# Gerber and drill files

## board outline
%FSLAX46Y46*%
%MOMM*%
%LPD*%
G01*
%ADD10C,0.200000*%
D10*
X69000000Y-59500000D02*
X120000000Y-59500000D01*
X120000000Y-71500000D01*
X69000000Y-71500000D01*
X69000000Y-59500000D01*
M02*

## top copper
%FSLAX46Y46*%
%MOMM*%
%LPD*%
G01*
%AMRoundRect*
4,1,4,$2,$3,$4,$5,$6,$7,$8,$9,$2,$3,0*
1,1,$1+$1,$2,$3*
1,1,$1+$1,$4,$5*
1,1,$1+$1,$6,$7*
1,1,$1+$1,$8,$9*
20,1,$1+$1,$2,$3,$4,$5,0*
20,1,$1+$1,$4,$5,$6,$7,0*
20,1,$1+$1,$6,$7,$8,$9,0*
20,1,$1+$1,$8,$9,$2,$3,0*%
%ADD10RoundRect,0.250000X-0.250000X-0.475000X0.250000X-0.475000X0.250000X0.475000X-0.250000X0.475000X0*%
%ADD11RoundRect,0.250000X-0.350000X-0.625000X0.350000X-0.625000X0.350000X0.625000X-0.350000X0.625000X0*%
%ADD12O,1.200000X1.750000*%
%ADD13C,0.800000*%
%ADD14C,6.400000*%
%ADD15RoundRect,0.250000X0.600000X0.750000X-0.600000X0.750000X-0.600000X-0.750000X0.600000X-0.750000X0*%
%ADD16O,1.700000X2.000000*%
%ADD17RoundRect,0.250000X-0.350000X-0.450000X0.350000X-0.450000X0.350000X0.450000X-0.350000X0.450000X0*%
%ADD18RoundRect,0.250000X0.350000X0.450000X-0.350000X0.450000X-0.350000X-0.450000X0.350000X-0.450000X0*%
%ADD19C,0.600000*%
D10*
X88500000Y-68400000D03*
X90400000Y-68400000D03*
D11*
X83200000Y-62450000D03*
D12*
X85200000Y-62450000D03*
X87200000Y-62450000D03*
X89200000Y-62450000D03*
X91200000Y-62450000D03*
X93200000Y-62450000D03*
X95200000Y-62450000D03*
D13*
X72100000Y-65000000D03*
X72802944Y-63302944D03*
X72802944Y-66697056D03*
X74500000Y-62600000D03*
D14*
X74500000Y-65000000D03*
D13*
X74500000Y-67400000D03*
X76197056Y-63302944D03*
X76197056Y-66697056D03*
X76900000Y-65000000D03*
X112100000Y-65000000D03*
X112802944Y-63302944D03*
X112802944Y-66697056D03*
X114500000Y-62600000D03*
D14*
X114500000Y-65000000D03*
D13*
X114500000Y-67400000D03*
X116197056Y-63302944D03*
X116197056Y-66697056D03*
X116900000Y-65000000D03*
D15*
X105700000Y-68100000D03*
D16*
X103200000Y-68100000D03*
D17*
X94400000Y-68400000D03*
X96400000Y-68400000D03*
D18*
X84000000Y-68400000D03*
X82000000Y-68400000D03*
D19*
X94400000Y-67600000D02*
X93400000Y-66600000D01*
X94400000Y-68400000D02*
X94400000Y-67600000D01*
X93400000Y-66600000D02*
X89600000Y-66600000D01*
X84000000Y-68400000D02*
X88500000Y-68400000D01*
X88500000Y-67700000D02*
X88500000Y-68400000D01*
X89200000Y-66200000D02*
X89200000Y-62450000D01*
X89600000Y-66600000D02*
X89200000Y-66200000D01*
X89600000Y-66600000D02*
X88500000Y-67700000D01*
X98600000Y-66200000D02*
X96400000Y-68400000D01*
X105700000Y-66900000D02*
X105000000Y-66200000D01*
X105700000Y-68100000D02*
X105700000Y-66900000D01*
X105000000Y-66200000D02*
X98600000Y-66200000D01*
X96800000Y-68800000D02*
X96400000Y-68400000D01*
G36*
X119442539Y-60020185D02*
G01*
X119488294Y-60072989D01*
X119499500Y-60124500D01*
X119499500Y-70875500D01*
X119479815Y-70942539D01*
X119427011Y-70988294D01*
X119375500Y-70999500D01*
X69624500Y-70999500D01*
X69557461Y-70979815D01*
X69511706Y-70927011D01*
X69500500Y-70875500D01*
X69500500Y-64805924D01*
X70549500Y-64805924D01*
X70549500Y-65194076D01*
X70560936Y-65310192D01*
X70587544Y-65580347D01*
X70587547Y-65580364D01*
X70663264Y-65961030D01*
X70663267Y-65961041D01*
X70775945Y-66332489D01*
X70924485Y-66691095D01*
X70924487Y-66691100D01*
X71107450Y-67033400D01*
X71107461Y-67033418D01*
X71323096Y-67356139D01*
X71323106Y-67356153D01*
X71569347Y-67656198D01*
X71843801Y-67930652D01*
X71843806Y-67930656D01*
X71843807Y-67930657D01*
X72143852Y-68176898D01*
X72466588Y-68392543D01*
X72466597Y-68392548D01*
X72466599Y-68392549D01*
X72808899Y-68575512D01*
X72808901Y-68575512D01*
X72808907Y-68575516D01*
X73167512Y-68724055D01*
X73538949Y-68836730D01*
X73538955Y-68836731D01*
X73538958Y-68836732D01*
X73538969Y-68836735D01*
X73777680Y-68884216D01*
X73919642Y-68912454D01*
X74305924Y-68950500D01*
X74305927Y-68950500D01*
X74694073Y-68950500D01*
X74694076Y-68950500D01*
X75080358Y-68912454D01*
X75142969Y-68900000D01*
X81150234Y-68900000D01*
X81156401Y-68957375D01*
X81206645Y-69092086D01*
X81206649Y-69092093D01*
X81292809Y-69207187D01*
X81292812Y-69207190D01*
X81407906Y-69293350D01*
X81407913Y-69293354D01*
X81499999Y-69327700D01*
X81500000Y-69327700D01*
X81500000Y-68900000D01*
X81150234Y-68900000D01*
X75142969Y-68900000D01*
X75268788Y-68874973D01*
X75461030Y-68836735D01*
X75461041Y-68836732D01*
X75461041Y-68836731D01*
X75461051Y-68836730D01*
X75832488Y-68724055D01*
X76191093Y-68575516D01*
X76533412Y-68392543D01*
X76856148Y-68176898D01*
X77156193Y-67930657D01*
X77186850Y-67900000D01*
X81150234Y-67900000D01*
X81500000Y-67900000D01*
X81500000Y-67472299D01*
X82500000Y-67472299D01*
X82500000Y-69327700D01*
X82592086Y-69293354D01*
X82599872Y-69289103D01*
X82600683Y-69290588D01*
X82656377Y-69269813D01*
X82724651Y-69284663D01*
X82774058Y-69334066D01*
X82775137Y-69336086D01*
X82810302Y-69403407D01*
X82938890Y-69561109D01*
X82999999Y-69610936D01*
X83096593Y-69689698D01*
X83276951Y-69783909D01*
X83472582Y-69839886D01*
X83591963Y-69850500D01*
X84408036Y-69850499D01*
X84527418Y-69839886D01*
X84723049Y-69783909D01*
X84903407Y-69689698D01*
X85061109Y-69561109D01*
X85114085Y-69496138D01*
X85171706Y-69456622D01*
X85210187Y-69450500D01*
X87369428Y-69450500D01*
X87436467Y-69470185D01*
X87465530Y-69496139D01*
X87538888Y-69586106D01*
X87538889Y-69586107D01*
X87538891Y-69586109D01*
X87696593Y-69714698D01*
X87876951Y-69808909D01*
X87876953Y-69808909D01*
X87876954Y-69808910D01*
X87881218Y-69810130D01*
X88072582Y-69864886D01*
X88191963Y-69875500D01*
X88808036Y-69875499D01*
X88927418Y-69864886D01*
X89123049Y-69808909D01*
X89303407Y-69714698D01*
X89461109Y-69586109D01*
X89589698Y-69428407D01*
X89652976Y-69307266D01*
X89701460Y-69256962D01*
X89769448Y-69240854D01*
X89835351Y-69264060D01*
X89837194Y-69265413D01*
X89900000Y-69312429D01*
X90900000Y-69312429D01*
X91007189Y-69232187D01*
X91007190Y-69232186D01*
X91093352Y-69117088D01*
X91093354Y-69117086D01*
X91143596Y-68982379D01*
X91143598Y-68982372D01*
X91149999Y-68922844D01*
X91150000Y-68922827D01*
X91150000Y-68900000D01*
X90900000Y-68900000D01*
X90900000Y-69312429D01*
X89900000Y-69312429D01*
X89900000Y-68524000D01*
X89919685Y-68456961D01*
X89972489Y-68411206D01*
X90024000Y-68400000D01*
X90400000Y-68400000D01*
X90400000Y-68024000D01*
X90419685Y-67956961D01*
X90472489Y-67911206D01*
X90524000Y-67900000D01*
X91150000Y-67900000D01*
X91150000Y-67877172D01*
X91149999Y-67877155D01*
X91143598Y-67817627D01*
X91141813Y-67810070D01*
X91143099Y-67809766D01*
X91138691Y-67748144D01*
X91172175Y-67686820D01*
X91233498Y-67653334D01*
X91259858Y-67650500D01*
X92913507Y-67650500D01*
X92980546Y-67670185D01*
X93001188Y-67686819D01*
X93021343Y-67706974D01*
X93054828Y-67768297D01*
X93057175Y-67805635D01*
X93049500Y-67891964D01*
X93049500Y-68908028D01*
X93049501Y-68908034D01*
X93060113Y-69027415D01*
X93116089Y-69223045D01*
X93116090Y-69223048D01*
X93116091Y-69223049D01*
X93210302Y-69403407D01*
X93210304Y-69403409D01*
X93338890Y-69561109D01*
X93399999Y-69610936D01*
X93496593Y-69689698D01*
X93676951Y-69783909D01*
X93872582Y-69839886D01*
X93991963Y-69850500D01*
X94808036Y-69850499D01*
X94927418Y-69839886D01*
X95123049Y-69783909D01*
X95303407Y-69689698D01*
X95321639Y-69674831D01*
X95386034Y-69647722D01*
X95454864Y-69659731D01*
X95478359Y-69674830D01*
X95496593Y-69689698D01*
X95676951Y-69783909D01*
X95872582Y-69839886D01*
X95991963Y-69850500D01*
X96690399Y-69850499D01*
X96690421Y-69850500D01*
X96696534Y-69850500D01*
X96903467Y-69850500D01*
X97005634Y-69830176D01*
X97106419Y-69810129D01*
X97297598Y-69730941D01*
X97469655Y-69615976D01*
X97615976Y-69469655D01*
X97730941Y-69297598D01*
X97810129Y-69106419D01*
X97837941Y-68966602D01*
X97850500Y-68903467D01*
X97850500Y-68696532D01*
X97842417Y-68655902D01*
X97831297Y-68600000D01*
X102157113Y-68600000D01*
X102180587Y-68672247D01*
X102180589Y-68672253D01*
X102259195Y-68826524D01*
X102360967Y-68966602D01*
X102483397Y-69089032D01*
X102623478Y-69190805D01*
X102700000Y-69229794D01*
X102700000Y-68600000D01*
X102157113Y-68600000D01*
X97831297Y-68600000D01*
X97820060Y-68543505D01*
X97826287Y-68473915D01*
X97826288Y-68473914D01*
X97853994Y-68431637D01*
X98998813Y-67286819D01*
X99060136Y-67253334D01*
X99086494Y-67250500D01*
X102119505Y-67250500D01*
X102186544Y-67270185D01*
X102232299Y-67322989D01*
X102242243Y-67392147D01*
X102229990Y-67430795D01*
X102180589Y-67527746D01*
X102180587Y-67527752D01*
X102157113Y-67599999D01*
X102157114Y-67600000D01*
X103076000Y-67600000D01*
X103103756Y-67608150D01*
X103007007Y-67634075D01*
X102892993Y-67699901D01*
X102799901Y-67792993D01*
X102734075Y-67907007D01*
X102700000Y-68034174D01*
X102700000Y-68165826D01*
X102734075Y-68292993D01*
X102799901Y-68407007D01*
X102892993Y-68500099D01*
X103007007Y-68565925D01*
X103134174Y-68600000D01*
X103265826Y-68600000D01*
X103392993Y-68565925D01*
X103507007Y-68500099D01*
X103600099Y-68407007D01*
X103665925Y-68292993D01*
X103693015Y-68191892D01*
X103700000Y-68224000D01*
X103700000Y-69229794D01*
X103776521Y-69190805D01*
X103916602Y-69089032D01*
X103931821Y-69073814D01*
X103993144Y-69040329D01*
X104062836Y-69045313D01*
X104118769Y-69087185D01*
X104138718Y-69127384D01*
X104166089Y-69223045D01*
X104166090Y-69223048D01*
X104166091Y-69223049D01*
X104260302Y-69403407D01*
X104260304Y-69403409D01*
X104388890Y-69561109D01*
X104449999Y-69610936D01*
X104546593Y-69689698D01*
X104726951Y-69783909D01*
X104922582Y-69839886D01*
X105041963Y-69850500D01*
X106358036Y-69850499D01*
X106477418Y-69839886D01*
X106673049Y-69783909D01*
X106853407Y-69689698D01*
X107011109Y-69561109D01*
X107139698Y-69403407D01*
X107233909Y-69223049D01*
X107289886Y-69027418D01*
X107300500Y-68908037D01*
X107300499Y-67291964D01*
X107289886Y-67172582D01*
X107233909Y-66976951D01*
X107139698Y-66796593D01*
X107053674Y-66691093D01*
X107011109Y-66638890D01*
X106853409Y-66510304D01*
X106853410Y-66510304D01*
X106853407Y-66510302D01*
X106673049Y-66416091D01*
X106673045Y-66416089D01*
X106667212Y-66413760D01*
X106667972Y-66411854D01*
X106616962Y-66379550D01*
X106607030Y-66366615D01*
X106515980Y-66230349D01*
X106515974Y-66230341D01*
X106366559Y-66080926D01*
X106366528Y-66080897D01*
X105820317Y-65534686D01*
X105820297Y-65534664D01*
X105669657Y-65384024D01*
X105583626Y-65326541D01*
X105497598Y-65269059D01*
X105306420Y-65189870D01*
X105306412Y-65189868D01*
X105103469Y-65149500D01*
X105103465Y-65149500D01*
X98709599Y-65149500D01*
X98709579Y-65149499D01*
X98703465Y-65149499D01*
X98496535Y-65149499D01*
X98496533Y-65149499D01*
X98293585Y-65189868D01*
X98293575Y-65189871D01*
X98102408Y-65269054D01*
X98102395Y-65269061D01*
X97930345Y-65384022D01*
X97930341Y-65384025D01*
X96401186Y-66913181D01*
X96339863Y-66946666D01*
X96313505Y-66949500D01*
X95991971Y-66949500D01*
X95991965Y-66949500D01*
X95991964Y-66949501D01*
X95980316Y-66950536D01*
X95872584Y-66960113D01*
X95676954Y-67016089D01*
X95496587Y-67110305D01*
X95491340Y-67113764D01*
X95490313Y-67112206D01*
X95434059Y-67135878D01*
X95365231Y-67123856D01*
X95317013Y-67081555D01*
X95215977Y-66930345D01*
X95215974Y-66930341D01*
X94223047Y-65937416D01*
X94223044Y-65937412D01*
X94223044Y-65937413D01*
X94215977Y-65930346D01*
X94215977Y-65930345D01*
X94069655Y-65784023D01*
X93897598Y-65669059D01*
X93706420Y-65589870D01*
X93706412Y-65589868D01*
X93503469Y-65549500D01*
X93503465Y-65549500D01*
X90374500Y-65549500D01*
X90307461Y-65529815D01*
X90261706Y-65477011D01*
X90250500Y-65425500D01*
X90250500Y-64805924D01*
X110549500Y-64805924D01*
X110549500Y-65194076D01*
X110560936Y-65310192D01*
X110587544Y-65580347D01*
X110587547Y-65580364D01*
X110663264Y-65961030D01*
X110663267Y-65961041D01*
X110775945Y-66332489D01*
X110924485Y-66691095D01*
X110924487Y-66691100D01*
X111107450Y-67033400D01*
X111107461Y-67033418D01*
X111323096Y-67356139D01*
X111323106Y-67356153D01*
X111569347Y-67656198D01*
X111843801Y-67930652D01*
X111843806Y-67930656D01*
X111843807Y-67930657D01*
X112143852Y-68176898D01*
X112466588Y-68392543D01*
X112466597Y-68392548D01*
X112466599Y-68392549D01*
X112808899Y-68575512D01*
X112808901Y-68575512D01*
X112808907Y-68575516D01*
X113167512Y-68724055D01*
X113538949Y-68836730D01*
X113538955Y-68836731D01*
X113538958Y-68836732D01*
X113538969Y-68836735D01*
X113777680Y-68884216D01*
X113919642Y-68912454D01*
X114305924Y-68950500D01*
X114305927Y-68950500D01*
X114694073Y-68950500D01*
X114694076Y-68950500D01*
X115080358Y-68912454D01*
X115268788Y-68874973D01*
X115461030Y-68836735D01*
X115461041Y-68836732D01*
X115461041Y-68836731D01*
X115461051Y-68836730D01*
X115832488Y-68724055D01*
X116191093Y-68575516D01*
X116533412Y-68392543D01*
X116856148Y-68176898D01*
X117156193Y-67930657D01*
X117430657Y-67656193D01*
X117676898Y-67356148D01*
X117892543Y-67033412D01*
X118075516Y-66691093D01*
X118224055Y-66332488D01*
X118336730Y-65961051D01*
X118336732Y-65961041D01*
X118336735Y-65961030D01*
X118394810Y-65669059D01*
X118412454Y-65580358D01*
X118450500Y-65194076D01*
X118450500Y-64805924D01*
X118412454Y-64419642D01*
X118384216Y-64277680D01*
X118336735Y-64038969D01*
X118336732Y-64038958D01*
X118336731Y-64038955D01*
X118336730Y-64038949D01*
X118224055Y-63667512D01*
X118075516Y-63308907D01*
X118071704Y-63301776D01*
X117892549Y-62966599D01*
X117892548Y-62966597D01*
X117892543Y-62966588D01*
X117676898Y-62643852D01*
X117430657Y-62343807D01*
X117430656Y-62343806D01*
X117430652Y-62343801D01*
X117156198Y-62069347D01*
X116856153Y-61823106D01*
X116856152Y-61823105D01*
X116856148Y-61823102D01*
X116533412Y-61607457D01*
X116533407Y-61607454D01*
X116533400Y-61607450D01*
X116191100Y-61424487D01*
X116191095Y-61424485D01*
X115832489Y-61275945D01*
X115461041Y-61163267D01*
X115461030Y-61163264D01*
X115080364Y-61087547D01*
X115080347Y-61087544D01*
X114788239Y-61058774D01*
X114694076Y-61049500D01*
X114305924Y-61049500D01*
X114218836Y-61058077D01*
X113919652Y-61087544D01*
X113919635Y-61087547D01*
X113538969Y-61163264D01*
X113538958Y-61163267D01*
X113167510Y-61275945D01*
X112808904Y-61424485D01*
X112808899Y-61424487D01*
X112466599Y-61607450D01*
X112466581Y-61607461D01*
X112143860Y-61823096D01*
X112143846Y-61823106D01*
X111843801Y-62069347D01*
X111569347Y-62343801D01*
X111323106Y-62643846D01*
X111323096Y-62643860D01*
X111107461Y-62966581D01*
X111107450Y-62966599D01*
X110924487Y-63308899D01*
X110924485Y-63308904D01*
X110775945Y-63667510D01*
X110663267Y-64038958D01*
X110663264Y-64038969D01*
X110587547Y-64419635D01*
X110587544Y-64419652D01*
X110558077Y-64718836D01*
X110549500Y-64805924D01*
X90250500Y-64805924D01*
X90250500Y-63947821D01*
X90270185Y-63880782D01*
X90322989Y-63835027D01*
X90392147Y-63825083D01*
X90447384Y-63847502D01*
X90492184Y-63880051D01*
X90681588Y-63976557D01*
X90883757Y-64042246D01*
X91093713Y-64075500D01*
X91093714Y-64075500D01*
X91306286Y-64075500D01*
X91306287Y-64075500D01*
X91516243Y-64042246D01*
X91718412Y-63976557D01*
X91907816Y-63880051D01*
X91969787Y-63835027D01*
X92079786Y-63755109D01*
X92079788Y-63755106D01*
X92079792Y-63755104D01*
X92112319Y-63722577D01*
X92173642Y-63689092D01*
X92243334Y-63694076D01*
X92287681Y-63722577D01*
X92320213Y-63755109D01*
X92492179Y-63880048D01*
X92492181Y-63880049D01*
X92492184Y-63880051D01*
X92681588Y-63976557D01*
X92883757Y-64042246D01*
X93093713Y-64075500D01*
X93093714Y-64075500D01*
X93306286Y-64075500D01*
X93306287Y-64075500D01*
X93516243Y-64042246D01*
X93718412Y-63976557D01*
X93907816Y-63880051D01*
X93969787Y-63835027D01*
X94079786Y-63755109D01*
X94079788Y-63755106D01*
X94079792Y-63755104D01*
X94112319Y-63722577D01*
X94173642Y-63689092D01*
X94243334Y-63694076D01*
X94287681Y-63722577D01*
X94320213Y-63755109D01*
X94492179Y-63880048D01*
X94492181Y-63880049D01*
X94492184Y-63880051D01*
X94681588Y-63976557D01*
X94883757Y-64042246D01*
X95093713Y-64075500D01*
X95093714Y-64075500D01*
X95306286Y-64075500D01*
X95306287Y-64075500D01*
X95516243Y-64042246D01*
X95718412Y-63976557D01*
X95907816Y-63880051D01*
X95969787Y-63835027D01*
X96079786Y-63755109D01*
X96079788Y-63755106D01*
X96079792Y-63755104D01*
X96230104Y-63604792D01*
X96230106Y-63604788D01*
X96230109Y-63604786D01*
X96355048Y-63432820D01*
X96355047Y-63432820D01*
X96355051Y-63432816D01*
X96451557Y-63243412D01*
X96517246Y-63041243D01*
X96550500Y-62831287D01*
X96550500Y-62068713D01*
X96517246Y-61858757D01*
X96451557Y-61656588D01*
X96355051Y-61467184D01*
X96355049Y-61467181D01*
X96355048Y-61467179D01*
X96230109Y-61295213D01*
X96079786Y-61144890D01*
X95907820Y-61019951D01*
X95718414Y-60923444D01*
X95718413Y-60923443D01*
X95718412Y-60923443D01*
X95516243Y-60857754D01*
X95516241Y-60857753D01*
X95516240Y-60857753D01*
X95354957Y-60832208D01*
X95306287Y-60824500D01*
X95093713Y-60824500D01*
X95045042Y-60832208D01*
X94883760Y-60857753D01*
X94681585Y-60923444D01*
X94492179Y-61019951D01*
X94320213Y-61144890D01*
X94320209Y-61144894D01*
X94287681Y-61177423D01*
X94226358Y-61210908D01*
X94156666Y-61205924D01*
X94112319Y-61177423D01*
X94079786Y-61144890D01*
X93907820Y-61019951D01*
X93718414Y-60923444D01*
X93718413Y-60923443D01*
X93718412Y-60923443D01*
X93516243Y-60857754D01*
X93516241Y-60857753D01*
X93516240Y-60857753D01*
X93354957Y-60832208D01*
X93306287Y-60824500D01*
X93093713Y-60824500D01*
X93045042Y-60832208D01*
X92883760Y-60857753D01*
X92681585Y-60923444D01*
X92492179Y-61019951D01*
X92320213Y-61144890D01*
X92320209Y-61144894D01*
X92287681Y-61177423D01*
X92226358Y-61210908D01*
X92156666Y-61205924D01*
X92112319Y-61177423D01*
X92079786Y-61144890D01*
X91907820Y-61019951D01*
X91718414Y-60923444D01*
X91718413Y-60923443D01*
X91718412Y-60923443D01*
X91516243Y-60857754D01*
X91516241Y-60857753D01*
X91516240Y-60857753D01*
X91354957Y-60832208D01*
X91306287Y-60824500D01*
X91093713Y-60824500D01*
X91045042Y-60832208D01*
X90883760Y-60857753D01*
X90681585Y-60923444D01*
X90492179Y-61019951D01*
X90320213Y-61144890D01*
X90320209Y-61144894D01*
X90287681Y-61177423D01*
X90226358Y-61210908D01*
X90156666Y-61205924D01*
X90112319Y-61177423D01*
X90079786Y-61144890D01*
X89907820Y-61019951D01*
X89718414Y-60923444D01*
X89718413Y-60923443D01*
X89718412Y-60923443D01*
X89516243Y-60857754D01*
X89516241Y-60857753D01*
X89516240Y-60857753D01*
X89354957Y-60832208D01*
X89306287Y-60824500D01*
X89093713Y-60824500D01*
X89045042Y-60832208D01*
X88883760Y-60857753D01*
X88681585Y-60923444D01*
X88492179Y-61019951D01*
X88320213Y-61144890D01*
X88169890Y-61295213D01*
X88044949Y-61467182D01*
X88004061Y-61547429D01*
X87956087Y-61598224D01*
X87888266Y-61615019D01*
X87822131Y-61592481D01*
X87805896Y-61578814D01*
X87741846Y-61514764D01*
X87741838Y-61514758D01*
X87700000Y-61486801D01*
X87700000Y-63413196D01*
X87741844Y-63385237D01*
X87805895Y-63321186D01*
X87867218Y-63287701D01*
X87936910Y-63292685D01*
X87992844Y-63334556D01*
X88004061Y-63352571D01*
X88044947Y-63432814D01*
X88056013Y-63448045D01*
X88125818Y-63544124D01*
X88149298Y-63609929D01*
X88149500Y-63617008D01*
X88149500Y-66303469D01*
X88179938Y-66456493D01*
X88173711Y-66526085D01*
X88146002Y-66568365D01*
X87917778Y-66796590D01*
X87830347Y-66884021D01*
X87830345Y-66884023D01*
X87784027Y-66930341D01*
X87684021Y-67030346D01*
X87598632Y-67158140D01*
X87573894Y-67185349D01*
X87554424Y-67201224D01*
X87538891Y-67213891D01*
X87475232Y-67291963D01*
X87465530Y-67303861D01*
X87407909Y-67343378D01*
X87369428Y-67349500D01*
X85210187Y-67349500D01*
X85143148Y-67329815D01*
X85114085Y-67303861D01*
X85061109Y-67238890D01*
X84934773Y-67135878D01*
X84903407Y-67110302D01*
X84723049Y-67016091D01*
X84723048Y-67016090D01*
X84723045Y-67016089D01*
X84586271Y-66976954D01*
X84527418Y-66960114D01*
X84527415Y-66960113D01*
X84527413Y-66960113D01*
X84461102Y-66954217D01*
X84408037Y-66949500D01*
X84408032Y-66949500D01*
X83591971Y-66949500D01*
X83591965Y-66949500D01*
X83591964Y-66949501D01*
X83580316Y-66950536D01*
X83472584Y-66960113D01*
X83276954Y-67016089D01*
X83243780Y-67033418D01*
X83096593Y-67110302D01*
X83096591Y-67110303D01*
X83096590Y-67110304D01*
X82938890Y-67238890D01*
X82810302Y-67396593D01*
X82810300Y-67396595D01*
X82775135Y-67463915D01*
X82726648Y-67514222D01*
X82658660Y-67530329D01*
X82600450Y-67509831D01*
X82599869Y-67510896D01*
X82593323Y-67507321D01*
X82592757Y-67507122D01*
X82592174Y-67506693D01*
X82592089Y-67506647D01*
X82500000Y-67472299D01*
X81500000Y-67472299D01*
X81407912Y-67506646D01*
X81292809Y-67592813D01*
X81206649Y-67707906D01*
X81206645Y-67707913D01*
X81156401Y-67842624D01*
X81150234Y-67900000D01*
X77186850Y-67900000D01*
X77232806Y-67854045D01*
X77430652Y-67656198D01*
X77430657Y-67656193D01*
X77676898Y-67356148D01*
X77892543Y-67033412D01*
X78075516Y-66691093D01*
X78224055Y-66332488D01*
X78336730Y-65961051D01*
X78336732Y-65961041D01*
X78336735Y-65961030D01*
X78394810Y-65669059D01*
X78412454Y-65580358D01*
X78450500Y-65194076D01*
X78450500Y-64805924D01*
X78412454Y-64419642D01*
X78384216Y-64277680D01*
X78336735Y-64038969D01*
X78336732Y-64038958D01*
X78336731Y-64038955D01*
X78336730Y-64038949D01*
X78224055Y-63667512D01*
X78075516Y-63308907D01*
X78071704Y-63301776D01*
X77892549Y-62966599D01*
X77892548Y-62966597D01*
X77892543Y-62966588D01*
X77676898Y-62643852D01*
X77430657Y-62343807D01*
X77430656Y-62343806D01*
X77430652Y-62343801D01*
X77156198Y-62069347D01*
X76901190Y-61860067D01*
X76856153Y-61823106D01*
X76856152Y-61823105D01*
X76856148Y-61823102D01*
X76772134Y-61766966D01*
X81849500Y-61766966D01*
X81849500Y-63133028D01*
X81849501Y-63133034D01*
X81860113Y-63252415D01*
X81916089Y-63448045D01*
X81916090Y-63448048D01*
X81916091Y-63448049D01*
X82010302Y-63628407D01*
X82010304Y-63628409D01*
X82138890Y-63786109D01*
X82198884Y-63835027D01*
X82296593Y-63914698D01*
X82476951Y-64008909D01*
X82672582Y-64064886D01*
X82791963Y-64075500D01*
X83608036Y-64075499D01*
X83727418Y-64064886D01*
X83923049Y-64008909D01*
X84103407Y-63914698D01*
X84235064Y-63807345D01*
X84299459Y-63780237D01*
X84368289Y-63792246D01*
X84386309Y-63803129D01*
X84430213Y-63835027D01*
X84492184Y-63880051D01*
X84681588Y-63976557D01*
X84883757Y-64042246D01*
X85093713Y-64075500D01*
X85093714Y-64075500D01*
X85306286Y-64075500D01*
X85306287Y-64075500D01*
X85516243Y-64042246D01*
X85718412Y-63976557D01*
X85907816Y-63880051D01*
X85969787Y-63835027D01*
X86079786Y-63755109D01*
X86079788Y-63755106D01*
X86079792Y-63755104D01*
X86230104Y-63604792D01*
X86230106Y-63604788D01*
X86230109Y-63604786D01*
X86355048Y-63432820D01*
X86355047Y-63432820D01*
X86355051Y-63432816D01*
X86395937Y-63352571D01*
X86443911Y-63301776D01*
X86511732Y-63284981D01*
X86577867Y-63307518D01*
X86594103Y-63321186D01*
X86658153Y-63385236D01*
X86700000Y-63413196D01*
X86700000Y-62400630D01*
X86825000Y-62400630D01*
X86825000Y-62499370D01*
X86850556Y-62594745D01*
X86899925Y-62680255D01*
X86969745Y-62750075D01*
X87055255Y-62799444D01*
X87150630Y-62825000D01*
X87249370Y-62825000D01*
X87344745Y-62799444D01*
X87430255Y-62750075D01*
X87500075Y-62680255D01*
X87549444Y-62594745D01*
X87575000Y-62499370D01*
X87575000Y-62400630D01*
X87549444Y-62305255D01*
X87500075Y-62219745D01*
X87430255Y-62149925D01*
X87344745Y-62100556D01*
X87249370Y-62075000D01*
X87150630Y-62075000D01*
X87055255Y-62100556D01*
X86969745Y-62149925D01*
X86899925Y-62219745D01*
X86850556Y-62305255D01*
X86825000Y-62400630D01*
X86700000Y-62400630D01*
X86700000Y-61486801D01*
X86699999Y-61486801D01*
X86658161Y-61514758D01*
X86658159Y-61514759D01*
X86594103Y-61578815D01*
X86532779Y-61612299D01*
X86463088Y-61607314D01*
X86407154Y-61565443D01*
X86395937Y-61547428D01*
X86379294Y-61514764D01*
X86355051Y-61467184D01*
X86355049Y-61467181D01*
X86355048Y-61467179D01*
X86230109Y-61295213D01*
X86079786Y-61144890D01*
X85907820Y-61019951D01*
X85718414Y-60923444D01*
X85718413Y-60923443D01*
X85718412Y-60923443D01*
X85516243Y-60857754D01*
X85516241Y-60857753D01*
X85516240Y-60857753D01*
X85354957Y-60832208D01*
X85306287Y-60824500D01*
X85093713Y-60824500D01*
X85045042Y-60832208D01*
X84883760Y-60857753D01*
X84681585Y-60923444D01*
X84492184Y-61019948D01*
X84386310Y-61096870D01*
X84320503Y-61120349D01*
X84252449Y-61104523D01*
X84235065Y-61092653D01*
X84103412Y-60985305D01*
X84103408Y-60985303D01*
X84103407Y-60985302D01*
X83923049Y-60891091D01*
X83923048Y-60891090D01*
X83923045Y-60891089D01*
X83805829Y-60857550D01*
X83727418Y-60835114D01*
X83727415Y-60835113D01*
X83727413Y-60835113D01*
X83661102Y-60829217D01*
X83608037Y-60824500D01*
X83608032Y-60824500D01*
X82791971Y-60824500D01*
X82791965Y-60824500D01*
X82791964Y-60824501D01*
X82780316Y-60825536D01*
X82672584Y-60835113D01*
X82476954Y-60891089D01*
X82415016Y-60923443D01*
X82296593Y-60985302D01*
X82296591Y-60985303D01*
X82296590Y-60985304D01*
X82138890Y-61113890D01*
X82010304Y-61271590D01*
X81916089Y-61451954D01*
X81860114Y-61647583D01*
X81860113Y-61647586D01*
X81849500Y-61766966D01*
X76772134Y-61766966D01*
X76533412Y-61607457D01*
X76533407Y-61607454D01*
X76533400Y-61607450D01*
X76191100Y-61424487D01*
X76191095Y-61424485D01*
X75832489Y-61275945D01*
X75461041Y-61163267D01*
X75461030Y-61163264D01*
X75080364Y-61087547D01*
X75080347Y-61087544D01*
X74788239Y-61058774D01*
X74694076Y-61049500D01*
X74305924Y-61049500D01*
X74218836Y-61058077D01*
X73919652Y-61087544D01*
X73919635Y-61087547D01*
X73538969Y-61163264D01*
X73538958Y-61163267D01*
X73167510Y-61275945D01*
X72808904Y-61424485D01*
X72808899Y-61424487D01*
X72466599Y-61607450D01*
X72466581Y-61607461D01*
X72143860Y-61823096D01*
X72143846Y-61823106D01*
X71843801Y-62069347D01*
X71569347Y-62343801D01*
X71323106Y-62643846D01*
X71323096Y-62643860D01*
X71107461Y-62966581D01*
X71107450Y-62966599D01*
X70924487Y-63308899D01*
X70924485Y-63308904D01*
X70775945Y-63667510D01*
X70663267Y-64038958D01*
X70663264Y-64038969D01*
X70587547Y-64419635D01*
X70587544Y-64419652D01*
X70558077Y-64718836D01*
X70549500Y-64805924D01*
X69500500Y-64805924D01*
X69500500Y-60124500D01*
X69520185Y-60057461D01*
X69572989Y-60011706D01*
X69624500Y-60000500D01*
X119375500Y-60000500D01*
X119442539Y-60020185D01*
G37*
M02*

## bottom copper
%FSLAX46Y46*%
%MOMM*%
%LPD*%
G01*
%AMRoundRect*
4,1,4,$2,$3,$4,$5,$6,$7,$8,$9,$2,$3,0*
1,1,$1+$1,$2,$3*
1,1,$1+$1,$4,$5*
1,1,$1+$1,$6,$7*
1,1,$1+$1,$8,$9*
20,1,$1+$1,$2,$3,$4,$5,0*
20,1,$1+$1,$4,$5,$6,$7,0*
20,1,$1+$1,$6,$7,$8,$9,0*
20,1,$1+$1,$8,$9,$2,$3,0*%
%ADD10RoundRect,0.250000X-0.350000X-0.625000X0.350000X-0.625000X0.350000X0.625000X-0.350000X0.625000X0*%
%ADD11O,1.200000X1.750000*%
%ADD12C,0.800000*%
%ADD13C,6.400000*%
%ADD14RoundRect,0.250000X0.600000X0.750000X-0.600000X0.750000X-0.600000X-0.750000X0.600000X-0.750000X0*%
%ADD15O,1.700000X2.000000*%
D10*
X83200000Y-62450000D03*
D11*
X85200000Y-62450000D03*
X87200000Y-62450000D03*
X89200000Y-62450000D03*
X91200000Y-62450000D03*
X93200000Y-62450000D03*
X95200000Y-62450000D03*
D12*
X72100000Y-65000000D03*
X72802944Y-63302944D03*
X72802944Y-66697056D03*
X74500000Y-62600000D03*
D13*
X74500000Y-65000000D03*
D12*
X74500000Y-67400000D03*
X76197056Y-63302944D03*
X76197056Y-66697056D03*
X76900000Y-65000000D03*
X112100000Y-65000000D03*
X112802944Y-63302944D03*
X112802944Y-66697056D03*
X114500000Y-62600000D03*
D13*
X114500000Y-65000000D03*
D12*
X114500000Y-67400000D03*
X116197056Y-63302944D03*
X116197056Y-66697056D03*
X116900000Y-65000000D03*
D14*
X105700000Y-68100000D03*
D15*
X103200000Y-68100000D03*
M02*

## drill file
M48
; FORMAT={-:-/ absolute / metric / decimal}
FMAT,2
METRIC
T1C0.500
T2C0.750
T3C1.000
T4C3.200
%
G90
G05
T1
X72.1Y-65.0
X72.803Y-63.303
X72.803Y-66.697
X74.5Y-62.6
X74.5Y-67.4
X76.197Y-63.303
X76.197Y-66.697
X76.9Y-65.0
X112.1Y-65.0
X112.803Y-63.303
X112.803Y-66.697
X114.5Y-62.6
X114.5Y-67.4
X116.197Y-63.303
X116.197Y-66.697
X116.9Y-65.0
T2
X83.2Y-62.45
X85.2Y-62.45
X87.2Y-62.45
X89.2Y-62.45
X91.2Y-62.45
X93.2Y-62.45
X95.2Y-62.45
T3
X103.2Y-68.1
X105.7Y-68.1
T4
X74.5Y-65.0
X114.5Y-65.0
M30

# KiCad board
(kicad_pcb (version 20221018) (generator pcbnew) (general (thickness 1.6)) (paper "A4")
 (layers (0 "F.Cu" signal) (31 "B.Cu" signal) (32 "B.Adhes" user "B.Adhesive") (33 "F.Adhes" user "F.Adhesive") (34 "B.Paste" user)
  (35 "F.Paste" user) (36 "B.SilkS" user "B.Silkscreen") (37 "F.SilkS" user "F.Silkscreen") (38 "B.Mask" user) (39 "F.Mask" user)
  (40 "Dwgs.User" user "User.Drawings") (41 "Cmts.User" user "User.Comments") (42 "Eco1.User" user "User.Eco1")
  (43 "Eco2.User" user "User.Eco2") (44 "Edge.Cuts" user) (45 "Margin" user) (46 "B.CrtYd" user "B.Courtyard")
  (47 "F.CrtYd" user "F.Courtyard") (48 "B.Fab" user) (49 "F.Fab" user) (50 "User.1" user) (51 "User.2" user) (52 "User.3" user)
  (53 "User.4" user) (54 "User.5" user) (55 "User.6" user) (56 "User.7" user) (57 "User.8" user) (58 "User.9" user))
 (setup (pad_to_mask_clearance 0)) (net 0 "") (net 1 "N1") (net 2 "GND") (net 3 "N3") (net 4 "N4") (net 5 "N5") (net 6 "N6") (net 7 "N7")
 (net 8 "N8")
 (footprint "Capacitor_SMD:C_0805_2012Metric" (layer "F.Cu") (at 89.45 68.4)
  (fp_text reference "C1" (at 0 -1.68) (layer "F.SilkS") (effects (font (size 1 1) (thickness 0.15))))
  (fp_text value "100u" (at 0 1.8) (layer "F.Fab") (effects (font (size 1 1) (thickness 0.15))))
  (pad "1" smd roundrect (at -0.95 0) (size 1 1.45) (layers "F.Cu" "F.Paste" "F.Mask") (roundrect_rratio 0.25) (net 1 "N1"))
  (pad "2" smd roundrect (at 0.95 0) (size 1 1.45) (layers "F.Cu" "F.Paste" "F.Mask") (roundrect_rratio 0.25) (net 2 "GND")))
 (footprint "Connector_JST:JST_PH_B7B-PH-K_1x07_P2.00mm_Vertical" (layer "F.Cu") (at 83.2 62.45)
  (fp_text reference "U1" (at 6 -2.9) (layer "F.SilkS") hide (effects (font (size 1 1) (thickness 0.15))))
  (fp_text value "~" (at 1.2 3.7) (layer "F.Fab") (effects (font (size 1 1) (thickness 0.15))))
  (pad "1" thru_hole roundrect (at 0 0) (size 1.2 1.75) (drill 0.75) (layers "*.Cu" "*.Mask") (roundrect_rratio 0.208333) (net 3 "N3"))
  (pad "2" thru_hole oval (at 2 0) (size 1.2 1.75) (drill 0.75) (layers "*.Cu" "*.Mask") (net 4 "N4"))
  (pad "3" thru_hole oval (at 4 0) (size 1.2 1.75) (drill 0.75) (layers "*.Cu" "*.Mask") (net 2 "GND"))
  (pad "4" thru_hole oval (at 6 0) (size 1.2 1.75) (drill 0.75) (layers "*.Cu" "*.Mask") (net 1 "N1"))
  (pad "5" thru_hole oval (at 8 0) (size 1.2 1.75) (drill 0.75) (layers "*.Cu" "*.Mask") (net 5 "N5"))
  (pad "6" thru_hole oval (at 10 0) (size 1.2 1.75) (drill 0.75) (layers "*.Cu" "*.Mask") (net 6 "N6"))
  (pad "7" thru_hole oval (at 12 0) (size 1.2 1.75) (drill 0.75) (layers "*.Cu" "*.Mask") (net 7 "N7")))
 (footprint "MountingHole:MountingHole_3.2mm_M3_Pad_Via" (layer "F.Cu") (at 74.5 65)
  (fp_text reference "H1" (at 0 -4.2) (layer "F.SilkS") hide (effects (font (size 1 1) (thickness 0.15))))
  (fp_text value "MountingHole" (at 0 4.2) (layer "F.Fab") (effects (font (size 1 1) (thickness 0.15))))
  (pad "1" thru_hole circle (at -2.4 0) (size 0.8 0.8) (drill 0.5) (layers "*.Cu" "*.Mask"))
  (pad "1" thru_hole circle (at -1.697056 -1.697056) (size 0.8 0.8) (drill 0.5) (layers "*.Cu" "*.Mask"))
  (pad "1" thru_hole circle (at -1.697056 1.697056) (size 0.8 0.8) (drill 0.5) (layers "*.Cu" "*.Mask"))
  (pad "1" thru_hole circle (at 0 -2.4) (size 0.8 0.8) (drill 0.5) (layers "*.Cu" "*.Mask"))
  (pad "1" thru_hole circle (at 0 0) (size 6.4 6.4) (drill 3.2) (layers "*.Cu" "*.Mask"))
  (pad "1" thru_hole circle (at 0 2.4) (size 0.8 0.8) (drill 0.5) (layers "*.Cu" "*.Mask"))
  (pad "1" thru_hole circle (at 1.697056 -1.697056) (size 0.8 0.8) (drill 0.5) (layers "*.Cu" "*.Mask"))
  (pad "1" thru_hole circle (at 1.697056 1.697056) (size 0.8 0.8) (drill 0.5) (layers "*.Cu" "*.Mask"))
  (pad "1" thru_hole circle (at 2.4 0) (size 0.8 0.8) (drill 0.5) (layers "*.Cu" "*.Mask")))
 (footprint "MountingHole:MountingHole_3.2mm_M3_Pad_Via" (layer "F.Cu") (at 114.5 65)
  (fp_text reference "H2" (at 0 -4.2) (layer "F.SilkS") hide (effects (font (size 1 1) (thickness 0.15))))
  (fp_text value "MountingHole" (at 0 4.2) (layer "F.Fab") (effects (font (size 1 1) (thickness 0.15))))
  (pad "1" thru_hole circle (at -2.4 0) (size 0.8 0.8) (drill 0.5) (layers "*.Cu" "*.Mask"))
  (pad "1" thru_hole circle (at -1.697056 -1.697056) (size 0.8 0.8) (drill 0.5) (layers "*.Cu" "*.Mask"))
  (pad "1" thru_hole circle (at -1.697056 1.697056) (size 0.8 0.8) (drill 0.5) (layers "*.Cu" "*.Mask"))
  (pad "1" thru_hole circle (at 0 -2.4) (size 0.8 0.8) (drill 0.5) (layers "*.Cu" "*.Mask"))
  (pad "1" thru_hole circle (at 0 0) (size 6.4 6.4) (drill 3.2) (layers "*.Cu" "*.Mask"))
  (pad "1" thru_hole circle (at 0 2.4) (size 0.8 0.8) (drill 0.5) (layers "*.Cu" "*.Mask"))
  (pad "1" thru_hole circle (at 1.697056 -1.697056) (size 0.8 0.8) (drill 0.5) (layers "*.Cu" "*.Mask"))
  (pad "1" thru_hole circle (at 1.697056 1.697056) (size 0.8 0.8) (drill 0.5) (layers "*.Cu" "*.Mask"))
  (pad "1" thru_hole circle (at 2.4 0) (size 0.8 0.8) (drill 0.5) (layers "*.Cu" "*.Mask")))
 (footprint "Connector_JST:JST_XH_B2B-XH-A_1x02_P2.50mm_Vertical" (layer "F.Cu") (at 105.7 68.1 180)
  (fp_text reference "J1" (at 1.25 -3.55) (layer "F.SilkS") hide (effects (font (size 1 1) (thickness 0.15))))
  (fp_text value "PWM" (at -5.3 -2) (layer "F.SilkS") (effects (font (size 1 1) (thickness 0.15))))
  (pad "1" thru_hole roundrect (at 0 0 180) (size 1.7 2) (drill 1) (layers "*.Cu" "*.Mask") (roundrect_rratio 0.147059) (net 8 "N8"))
  (pad "2" thru_hole oval (at 2.5 0 180) (size 1.7 2) (drill 1) (layers "*.Cu" "*.Mask") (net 2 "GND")))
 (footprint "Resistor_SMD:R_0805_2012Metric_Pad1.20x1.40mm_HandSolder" (layer "F.Cu") (at 95.4 68.4)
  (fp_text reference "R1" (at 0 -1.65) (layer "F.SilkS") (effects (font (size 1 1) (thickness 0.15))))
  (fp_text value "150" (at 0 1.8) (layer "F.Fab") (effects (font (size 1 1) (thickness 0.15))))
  (pad "1" smd roundrect (at -1 0) (size 1.2 1.4) (layers "F.Cu" "F.Paste" "F.Mask") (roundrect_rratio 0.208333) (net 1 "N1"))
  (pad "2" smd roundrect (at 1 0) (size 1.2 1.4) (layers "F.Cu" "F.Paste" "F.Mask") (roundrect_rratio 0.208333) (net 8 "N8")))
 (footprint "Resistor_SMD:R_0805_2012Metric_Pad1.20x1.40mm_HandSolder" (layer "F.Cu") (at 83 68.4 180)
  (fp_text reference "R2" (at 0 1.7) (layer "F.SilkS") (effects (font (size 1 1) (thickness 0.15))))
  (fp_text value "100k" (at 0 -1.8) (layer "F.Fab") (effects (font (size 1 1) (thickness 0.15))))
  (pad "1" smd roundrect (at -1 0 180) (size 1.2 1.4) (layers "F.Cu" "F.Paste" "F.Mask") (roundrect_rratio 0.208333) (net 1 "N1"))
  (pad "2" smd roundrect (at 1 0 180) (size 1.2 1.4) (layers "F.Cu" "F.Paste" "F.Mask") (roundrect_rratio 0.208333) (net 2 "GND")))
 (gr_rect (start 69 59.5) (end 120 71.5) (stroke (width 0.2) (type default)) (fill none) (layer "Edge.Cuts"))
 (segment (start 94.4 67.6) (end 93.4 66.6) (width 0.6) (layer "F.Cu") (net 1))
 (segment (start 94.4 68.4) (end 94.4 67.6) (width 0.6) (layer "F.Cu") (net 1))
 (segment (start 93.4 66.6) (end 89.6 66.6) (width 0.6) (layer "F.Cu") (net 1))
 (segment (start 84 68.4) (end 88.5 68.4) (width 0.6) (layer "F.Cu") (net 1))
 (segment (start 88.5 67.7) (end 88.5 68.4) (width 0.6) (layer "F.Cu") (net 1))
 (segment (start 89.2 66.2) (end 89.2 62.45) (width 0.6) (layer "F.Cu") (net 1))
 (segment (start 89.6 66.6) (end 89.2 66.2) (width 0.6) (layer "F.Cu") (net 1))
 (segment (start 89.6 66.6) (end 88.5 67.7) (width 0.6) (layer "F.Cu") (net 1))
 (segment (start 98.6 66.2) (end 96.4 68.4) (width 0.6) (layer "F.Cu") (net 8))
 (segment (start 105.7 66.9) (end 105 66.2) (width 0.6) (layer "F.Cu") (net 8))
 (segment (start 105.7 68.1) (end 105.7 66.9) (width 0.6) (layer "F.Cu") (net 8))
 (segment (start 105 66.2) (end 98.6 66.2) (width 0.6) (layer "F.Cu") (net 8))
 (segment (start 96.8 68.8) (end 96.4 68.4) (width 0.6) (layer "F.Cu") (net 8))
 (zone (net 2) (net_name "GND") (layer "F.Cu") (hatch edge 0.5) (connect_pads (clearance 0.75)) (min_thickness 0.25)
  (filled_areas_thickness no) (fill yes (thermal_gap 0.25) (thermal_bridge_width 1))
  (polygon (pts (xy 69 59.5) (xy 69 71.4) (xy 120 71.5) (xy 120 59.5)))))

